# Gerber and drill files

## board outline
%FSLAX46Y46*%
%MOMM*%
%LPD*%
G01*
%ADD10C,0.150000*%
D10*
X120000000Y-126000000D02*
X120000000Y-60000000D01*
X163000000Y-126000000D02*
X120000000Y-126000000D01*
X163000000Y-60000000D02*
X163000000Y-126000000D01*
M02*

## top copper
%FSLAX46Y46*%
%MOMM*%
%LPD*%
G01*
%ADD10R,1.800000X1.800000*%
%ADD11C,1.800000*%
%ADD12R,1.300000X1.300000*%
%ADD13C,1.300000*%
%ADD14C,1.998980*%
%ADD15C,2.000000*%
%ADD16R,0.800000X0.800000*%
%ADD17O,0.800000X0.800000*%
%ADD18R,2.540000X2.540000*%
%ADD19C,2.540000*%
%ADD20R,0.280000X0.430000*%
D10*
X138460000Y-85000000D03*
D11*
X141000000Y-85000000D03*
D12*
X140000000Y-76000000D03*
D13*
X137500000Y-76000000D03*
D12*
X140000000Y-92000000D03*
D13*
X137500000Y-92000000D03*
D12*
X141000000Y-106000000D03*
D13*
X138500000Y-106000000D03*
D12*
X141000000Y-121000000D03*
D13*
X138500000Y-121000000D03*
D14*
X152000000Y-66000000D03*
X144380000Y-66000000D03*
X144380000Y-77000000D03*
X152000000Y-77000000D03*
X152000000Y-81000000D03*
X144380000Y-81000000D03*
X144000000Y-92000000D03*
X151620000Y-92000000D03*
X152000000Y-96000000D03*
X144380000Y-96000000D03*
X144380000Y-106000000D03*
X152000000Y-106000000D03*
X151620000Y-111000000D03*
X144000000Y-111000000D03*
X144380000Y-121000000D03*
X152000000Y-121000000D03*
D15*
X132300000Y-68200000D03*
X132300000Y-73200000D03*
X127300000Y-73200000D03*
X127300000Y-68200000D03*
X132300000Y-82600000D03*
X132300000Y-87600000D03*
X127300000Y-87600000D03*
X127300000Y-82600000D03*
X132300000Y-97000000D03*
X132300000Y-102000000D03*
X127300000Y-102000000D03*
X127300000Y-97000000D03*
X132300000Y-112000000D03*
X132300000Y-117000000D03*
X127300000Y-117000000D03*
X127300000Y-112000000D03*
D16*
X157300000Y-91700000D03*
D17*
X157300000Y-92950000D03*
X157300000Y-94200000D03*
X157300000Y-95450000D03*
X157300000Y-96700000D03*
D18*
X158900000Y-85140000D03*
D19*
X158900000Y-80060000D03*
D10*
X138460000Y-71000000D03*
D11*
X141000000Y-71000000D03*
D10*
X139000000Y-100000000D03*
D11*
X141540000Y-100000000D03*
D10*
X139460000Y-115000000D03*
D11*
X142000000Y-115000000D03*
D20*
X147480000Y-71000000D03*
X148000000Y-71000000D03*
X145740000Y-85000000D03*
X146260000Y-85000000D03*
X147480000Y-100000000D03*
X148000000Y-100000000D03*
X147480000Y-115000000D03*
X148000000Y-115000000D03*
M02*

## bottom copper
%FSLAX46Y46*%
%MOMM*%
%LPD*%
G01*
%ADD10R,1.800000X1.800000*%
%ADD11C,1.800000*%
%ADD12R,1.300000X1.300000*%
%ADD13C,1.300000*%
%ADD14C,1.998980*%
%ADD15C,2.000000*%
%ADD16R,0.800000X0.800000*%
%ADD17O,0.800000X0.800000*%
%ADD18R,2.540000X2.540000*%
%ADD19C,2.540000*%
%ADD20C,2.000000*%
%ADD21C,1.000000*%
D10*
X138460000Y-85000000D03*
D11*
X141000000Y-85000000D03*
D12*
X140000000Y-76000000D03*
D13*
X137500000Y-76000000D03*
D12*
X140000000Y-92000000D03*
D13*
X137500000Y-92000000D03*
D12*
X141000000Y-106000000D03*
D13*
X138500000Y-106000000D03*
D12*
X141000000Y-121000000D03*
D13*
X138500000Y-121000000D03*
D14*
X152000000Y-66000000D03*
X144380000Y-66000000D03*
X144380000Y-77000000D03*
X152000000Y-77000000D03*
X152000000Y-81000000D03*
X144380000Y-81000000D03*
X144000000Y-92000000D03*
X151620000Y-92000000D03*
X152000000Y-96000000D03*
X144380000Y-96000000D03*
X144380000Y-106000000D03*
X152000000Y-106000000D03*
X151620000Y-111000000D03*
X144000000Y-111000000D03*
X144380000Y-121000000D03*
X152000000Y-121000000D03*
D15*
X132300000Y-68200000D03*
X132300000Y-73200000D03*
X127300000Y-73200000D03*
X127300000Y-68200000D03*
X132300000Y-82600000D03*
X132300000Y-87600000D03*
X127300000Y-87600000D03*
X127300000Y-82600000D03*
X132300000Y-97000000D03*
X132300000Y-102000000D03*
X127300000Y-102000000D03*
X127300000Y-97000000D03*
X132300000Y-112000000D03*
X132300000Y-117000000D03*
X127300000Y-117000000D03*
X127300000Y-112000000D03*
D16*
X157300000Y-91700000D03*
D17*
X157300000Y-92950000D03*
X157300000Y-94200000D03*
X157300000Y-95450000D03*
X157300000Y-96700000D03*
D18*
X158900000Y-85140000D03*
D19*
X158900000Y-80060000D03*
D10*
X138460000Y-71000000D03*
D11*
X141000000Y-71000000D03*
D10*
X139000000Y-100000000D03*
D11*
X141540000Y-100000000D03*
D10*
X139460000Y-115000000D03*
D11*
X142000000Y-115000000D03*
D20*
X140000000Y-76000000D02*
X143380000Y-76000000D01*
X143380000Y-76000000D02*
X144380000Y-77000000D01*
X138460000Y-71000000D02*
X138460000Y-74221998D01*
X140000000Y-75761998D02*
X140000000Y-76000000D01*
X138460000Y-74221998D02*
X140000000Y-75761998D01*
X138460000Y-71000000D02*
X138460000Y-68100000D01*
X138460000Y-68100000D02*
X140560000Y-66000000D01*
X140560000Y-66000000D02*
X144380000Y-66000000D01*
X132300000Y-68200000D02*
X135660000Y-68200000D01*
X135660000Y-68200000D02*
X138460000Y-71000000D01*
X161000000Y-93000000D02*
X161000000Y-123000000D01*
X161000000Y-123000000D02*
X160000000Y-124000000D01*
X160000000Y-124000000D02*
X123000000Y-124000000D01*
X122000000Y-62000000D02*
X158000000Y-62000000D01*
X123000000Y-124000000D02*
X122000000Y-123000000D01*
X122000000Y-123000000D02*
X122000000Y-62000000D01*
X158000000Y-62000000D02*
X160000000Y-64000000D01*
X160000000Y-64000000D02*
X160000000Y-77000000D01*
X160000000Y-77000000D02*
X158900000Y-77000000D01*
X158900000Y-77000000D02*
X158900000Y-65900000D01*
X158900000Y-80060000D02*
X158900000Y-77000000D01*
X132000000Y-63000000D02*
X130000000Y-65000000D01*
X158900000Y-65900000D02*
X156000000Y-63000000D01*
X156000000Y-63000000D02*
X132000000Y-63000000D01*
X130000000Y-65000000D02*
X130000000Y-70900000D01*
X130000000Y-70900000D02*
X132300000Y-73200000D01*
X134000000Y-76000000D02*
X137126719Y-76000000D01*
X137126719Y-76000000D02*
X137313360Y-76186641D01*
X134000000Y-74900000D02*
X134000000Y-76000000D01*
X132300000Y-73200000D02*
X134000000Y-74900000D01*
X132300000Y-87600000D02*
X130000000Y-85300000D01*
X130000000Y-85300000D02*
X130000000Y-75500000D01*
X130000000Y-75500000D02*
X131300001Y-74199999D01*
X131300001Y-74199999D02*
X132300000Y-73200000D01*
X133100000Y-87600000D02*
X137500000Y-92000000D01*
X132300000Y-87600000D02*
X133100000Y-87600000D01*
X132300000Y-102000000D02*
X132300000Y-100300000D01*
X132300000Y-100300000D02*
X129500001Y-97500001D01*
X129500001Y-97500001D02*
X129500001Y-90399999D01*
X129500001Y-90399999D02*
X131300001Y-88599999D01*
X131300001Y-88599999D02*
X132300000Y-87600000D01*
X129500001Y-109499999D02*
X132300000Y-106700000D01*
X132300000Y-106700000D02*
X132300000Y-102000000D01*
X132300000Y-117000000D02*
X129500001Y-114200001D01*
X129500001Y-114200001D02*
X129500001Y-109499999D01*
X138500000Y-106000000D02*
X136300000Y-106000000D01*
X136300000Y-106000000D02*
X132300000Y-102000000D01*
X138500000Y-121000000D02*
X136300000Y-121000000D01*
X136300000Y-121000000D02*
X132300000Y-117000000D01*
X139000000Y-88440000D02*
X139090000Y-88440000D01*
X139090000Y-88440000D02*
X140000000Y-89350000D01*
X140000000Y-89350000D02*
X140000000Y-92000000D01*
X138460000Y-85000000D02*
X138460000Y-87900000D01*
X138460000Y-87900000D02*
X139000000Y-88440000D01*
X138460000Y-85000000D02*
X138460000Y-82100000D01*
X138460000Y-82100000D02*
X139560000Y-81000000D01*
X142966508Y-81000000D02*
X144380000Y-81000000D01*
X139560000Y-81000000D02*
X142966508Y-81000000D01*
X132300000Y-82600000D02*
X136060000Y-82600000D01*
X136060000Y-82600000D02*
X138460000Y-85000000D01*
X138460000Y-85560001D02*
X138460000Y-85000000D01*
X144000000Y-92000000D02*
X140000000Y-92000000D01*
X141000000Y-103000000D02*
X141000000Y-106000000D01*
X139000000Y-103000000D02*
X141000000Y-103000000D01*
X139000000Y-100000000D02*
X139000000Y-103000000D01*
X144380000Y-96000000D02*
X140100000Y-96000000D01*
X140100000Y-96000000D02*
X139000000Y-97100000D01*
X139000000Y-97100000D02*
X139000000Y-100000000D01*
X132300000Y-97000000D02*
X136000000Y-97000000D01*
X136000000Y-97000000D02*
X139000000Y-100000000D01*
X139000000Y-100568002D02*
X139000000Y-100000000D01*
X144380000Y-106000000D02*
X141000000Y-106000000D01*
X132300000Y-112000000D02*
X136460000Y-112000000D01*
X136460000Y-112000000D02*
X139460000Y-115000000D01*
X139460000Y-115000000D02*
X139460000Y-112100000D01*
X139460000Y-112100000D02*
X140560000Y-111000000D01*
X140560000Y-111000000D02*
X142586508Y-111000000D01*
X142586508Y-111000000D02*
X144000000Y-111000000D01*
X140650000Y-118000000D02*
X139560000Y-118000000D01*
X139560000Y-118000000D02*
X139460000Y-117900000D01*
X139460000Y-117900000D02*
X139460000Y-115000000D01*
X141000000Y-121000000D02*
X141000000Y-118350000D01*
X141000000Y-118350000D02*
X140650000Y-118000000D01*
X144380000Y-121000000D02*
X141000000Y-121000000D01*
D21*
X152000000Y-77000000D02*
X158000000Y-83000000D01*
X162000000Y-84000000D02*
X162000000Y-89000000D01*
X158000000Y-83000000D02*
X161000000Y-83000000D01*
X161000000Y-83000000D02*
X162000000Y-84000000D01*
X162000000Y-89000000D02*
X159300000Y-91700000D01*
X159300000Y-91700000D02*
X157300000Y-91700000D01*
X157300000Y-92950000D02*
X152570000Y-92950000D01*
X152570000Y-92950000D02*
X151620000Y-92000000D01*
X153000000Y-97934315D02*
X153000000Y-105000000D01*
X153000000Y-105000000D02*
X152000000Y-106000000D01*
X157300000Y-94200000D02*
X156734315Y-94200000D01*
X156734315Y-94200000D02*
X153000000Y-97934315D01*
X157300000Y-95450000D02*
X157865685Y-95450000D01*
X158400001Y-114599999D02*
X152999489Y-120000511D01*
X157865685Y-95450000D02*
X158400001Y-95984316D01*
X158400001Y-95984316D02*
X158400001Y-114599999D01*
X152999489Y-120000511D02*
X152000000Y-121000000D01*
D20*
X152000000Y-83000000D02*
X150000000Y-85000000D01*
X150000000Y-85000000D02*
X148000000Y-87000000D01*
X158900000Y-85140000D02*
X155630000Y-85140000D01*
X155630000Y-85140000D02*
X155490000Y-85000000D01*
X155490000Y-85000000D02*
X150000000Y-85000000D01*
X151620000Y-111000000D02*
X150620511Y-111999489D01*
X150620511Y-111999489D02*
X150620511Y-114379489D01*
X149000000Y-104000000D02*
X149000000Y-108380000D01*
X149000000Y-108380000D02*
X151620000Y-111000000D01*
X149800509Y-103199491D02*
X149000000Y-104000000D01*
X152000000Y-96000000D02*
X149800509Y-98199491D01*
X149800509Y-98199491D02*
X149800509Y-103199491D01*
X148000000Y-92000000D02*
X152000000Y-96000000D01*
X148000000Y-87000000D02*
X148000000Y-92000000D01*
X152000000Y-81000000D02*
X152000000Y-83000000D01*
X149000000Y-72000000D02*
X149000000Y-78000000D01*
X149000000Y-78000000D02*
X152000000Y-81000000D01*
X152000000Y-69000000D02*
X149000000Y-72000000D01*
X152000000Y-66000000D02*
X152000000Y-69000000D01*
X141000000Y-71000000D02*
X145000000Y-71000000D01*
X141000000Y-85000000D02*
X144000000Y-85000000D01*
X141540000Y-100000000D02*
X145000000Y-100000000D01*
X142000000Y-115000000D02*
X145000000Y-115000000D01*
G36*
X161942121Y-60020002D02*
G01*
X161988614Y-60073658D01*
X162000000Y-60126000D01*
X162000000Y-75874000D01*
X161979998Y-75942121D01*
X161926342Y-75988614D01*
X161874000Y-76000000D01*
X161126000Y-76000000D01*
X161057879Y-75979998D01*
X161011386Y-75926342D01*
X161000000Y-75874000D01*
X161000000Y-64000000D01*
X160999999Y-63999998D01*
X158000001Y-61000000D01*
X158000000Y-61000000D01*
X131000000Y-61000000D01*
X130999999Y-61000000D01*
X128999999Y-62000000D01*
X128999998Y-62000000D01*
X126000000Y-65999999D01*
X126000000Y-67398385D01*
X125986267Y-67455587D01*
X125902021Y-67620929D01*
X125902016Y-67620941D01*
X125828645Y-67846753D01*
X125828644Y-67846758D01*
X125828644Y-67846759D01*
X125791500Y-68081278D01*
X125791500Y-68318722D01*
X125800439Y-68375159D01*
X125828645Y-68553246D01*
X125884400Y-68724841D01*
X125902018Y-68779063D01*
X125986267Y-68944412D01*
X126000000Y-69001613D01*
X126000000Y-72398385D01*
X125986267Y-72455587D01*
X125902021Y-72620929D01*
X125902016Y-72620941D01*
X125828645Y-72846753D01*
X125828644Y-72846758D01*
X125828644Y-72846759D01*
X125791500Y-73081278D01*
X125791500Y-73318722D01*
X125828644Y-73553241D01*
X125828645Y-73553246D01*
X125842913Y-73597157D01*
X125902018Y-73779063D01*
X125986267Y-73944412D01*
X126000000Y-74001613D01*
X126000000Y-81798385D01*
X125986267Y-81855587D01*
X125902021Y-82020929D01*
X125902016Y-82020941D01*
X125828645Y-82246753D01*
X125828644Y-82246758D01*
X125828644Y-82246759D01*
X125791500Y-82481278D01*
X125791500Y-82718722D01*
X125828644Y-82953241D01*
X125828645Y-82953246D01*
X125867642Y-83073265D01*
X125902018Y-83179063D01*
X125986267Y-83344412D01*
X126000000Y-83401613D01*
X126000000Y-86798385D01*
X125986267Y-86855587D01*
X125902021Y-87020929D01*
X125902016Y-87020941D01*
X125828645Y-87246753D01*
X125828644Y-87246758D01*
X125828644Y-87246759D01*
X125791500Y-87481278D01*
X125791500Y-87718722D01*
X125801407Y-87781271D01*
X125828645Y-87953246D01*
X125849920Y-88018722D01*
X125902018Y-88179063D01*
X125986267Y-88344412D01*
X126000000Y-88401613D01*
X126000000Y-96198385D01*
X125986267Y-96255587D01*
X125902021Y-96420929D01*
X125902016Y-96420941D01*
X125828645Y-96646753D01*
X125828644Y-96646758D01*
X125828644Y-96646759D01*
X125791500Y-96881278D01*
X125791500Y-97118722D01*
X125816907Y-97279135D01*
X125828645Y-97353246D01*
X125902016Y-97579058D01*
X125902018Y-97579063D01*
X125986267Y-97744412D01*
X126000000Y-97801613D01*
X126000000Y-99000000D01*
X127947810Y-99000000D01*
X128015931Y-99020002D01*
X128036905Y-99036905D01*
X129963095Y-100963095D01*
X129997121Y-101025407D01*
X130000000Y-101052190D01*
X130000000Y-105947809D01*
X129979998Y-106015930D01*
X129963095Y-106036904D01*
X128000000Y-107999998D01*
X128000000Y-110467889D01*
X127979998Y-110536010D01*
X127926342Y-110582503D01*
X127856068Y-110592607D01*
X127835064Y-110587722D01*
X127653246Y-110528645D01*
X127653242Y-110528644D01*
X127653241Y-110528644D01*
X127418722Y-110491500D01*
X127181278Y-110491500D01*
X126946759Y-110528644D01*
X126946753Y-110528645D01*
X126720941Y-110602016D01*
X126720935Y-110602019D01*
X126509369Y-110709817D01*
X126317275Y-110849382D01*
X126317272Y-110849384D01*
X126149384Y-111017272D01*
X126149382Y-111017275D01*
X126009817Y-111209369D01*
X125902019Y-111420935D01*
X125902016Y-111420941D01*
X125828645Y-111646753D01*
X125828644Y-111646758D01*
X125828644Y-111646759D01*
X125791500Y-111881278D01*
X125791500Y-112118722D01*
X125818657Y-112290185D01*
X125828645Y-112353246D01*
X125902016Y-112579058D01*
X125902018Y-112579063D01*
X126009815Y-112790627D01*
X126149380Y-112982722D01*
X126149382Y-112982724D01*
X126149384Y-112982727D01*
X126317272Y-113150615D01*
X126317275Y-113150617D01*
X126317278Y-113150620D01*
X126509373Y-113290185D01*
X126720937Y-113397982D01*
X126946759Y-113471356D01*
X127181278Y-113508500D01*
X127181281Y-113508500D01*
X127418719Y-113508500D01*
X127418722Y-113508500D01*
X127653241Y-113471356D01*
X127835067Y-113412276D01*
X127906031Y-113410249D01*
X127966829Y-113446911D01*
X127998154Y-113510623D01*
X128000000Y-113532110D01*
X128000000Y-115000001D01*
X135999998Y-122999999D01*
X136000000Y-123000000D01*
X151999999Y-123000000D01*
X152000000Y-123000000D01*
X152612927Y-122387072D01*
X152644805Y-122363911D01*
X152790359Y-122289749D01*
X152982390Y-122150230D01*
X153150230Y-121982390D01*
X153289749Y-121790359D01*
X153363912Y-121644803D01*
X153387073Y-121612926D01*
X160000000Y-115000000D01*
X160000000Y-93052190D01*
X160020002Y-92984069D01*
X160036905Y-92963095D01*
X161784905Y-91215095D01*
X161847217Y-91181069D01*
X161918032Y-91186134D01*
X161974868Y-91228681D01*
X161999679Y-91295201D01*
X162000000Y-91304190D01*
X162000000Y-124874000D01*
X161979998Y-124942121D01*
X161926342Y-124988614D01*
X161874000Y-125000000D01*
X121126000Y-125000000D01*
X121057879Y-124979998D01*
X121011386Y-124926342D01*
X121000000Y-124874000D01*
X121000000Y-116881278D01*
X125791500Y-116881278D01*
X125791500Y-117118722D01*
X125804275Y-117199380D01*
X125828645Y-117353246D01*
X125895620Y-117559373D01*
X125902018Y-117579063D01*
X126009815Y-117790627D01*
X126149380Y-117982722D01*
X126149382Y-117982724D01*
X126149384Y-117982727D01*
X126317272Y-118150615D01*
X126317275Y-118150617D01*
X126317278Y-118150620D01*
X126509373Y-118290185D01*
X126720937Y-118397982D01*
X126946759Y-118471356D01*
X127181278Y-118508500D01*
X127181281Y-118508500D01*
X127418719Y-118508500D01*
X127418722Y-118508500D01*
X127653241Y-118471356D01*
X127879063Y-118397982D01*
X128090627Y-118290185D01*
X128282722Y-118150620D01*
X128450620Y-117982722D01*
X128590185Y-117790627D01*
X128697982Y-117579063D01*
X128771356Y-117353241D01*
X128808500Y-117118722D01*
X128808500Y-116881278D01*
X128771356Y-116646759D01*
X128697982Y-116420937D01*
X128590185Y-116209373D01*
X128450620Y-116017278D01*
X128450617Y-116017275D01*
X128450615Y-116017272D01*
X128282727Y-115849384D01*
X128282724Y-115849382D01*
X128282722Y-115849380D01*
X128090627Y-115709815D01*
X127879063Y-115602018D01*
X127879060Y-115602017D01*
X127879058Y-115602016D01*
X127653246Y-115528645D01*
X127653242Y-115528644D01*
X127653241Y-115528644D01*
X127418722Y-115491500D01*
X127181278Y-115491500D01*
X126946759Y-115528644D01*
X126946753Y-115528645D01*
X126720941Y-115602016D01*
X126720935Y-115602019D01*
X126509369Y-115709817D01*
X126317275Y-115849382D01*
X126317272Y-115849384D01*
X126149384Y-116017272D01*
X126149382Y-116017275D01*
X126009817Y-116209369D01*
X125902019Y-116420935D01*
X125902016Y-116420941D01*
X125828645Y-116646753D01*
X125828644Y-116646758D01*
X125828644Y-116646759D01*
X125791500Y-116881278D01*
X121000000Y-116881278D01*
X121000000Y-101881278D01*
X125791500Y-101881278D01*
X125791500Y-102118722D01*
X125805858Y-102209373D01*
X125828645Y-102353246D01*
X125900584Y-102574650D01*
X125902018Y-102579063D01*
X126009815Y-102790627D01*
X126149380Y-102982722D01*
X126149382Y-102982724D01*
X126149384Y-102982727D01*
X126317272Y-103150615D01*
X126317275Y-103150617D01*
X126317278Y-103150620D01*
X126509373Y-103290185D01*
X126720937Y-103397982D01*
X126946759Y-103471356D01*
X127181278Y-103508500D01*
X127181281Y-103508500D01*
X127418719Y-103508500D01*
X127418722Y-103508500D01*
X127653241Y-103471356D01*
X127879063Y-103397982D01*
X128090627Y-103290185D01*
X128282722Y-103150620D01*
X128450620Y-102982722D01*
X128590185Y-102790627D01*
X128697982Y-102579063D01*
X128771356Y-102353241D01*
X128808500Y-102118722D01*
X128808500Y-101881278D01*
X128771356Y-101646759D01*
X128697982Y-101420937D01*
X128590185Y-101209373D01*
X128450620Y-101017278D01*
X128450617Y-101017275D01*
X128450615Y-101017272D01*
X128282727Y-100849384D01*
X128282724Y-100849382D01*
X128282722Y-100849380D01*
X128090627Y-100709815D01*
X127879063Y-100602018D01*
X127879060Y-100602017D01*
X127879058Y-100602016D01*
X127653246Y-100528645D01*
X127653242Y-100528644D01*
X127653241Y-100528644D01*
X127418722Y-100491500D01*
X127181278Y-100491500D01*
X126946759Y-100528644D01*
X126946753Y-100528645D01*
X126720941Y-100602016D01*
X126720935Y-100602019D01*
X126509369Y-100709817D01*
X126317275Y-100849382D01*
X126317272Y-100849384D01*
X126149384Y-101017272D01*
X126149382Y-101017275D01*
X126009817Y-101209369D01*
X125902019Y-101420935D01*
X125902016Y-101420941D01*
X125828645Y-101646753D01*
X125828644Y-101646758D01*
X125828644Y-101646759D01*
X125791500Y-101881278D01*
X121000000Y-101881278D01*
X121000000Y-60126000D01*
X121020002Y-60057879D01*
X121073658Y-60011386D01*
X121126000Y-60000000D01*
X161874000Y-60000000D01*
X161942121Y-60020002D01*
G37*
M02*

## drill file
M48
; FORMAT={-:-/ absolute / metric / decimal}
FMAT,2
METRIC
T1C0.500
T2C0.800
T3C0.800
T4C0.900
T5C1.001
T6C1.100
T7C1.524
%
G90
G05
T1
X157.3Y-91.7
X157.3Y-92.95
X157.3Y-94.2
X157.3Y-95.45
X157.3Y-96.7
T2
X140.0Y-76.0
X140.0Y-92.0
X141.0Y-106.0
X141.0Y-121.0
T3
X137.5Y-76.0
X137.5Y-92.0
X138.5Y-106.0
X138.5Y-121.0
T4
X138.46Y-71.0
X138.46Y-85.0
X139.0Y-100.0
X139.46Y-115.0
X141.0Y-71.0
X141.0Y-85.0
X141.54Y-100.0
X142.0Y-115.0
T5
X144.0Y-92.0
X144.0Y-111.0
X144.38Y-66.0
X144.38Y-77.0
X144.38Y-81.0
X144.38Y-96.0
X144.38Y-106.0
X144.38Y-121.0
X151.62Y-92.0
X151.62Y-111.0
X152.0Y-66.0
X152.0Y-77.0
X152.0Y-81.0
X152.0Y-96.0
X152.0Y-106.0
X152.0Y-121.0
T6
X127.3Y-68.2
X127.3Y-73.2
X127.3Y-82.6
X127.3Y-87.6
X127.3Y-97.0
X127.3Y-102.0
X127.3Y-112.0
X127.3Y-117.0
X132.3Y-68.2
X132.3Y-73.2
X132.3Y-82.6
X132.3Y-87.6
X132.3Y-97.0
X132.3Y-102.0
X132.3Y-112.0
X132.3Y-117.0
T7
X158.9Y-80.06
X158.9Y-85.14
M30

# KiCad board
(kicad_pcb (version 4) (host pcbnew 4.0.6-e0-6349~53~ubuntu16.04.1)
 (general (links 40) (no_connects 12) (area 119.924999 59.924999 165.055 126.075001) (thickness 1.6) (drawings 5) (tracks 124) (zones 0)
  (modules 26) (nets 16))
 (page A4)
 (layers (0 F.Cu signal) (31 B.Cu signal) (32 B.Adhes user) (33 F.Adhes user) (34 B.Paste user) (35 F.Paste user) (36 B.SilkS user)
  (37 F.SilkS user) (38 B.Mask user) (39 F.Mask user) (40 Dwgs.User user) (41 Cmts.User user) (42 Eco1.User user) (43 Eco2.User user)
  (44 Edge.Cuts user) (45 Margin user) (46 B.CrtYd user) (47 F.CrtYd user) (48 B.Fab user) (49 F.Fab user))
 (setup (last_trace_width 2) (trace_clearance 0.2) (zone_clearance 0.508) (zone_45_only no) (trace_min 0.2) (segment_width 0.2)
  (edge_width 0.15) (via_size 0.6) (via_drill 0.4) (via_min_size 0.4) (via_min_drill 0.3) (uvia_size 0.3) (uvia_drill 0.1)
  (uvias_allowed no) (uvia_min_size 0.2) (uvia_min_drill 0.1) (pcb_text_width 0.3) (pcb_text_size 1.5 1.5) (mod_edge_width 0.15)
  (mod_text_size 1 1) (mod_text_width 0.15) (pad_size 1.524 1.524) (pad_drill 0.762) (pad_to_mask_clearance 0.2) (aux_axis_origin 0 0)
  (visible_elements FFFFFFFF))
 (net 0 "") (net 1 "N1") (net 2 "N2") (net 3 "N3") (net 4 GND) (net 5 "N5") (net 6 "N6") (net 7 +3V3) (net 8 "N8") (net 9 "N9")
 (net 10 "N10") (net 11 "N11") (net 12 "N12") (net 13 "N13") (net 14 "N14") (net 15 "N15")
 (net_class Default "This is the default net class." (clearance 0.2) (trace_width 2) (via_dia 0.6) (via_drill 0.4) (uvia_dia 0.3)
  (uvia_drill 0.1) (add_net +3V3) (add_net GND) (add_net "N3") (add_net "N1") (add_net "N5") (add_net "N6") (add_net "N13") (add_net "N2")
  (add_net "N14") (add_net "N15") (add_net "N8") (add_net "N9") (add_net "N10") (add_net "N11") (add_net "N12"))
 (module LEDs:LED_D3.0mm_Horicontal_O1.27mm (layer F.Cu) (at 138.46 85)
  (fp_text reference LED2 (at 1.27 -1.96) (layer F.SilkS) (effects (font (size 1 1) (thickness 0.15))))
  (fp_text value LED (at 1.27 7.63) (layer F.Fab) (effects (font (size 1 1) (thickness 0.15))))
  (pad 1 thru_hole rect (at 0 0) (size 1.8 1.8) (drill 0.9) (layers *.Cu *.Mask) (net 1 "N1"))
  (pad 2 thru_hole circle (at 2.54 0) (size 1.8 1.8) (drill 0.9) (layers *.Cu *.Mask) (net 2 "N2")))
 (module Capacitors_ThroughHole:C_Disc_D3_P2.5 (layer F.Cu) (at 140 76 180)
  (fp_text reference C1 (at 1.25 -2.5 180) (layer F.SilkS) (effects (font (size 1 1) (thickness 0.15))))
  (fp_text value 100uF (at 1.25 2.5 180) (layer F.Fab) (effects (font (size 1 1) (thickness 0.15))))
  (pad 1 thru_hole rect (at 0 0 180) (size 1.3 1.3) (drill 0.8) (layers *.Cu *.Mask F.SilkS) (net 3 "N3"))
  (pad 2 thru_hole circle (at 2.5 0 180) (size 1.3 1.3) (drill 0.8001) (layers *.Cu *.Mask F.SilkS) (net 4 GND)))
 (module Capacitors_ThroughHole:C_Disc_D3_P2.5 (layer F.Cu) (at 140 92 180)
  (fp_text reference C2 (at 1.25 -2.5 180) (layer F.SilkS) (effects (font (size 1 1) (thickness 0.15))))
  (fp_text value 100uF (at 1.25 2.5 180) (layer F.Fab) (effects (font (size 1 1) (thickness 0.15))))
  (pad 1 thru_hole rect (at 0 0 180) (size 1.3 1.3) (drill 0.8) (layers *.Cu *.Mask F.SilkS) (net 1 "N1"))
  (pad 2 thru_hole circle (at 2.5 0 180) (size 1.3 1.3) (drill 0.8001) (layers *.Cu *.Mask F.SilkS) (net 4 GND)))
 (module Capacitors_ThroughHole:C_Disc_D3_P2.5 (layer F.Cu) (at 141 106 180)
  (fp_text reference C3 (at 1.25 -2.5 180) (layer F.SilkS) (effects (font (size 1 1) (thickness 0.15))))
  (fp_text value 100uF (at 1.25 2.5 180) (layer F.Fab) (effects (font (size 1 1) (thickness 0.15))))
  (pad 1 thru_hole rect (at 0 0 180) (size 1.3 1.3) (drill 0.8) (layers *.Cu *.Mask F.SilkS) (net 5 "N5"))
  (pad 2 thru_hole circle (at 2.5 0 180) (size 1.3 1.3) (drill 0.8001) (layers *.Cu *.Mask F.SilkS) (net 4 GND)))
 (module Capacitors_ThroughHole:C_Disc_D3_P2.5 (layer F.Cu) (at 141 121 180)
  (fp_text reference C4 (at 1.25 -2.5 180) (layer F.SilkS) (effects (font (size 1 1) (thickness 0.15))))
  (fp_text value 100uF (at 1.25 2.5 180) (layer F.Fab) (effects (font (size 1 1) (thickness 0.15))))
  (pad 1 thru_hole rect (at 0 0 180) (size 1.3 1.3) (drill 0.8) (layers *.Cu *.Mask F.SilkS) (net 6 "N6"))
  (pad 2 thru_hole circle (at 2.5 0 180) (size 1.3 1.3) (drill 0.8001) (layers *.Cu *.Mask F.SilkS) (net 4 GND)))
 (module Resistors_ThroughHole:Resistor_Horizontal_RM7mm (layer F.Cu) (at 152 66 180)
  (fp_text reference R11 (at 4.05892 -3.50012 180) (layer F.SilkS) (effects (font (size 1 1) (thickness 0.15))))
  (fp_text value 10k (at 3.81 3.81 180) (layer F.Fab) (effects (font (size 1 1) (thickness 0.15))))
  (pad 1 thru_hole circle (at 0 0 180) (size 1.99898 1.99898) (drill 1.00076) (layers *.Cu *.SilkS *.Mask) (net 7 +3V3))
  (pad 2 thru_hole circle (at 7.62 0 180) (size 1.99898 1.99898) (drill 1.00076) (layers *.Cu *.SilkS *.Mask) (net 3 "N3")))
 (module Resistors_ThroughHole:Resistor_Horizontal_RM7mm (layer F.Cu) (at 144.38 77)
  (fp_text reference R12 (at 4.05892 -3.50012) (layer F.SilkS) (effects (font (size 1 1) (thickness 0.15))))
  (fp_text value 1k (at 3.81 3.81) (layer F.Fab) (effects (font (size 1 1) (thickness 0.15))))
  (pad 1 thru_hole circle (at 0 0) (size 1.99898 1.99898) (drill 1.00076) (layers *.Cu *.SilkS *.Mask) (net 3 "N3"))
  (pad 2 thru_hole circle (at 7.62 0) (size 1.99898 1.99898) (drill 1.00076) (layers *.Cu *.SilkS *.Mask) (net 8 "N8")))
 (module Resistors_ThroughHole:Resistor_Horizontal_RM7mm (layer F.Cu) (at 152 81 180)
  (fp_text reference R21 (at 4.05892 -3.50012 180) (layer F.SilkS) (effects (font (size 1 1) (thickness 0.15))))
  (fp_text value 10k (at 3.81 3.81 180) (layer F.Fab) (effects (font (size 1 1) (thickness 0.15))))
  (pad 1 thru_hole circle (at 0 0 180) (size 1.99898 1.99898) (drill 1.00076) (layers *.Cu *.SilkS *.Mask) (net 7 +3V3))
  (pad 2 thru_hole circle (at 7.62 0 180) (size 1.99898 1.99898) (drill 1.00076) (layers *.Cu *.SilkS *.Mask) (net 1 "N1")))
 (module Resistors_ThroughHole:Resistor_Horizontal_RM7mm (layer F.Cu) (at 144 92)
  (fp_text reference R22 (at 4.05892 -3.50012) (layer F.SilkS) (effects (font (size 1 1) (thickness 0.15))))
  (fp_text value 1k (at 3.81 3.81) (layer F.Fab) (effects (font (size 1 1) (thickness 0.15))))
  (pad 1 thru_hole circle (at 0 0) (size 1.99898 1.99898) (drill 1.00076) (layers *.Cu *.SilkS *.Mask) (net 1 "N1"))
  (pad 2 thru_hole circle (at 7.62 0) (size 1.99898 1.99898) (drill 1.00076) (layers *.Cu *.SilkS *.Mask) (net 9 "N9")))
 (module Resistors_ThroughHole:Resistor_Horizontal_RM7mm (layer F.Cu) (at 152 96 180)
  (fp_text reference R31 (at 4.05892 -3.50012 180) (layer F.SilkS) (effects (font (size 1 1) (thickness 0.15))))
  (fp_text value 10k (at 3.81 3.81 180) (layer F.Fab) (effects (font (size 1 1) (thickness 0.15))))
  (pad 1 thru_hole circle (at 0 0 180) (size 1.99898 1.99898) (drill 1.00076) (layers *.Cu *.SilkS *.Mask) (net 7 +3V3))
  (pad 2 thru_hole circle (at 7.62 0 180) (size 1.99898 1.99898) (drill 1.00076) (layers *.Cu *.SilkS *.Mask) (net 5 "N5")))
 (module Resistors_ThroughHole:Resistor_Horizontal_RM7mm (layer F.Cu) (at 144.38 106)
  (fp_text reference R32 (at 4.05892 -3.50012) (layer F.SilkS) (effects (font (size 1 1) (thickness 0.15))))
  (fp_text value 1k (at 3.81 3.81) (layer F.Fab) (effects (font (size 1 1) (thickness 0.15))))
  (pad 1 thru_hole circle (at 0 0) (size 1.99898 1.99898) (drill 1.00076) (layers *.Cu *.SilkS *.Mask) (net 5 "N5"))
  (pad 2 thru_hole circle (at 7.62 0) (size 1.99898 1.99898) (drill 1.00076) (layers *.Cu *.SilkS *.Mask) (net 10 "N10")))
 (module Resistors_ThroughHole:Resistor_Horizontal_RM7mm (layer F.Cu) (at 151.62 111 180)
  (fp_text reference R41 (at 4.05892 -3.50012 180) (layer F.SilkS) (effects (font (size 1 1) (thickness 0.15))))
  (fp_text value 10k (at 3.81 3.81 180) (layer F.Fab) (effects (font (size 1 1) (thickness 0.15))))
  (pad 1 thru_hole circle (at 0 0 180) (size 1.99898 1.99898) (drill 1.00076) (layers *.Cu *.SilkS *.Mask) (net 7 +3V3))
  (pad 2 thru_hole circle (at 7.62 0 180) (size 1.99898 1.99898) (drill 1.00076) (layers *.Cu *.SilkS *.Mask) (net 6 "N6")))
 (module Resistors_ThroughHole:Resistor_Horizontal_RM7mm (layer F.Cu) (at 144.38 121)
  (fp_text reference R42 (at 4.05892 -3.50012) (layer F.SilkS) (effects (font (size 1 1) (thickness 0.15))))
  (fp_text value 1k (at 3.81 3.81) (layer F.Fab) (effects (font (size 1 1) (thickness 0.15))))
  (pad 1 thru_hole circle (at 0 0) (size 1.99898 1.99898) (drill 1.00076) (layers *.Cu *.SilkS *.Mask) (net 6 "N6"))
  (pad 2 thru_hole circle (at 7.62 0) (size 1.99898 1.99898) (drill 1.00076) (layers *.Cu *.SilkS *.Mask) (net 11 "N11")))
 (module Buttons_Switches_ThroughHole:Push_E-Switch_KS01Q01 (layer F.Cu) (at 132.3 68.2 270)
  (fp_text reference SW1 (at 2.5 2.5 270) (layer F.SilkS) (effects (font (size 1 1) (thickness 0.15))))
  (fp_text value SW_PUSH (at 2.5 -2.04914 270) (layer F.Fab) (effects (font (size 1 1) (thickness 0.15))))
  (pad 1 thru_hole circle (at 0 0 270) (size 2 2) (drill 1.1) (layers *.Cu *.Mask F.SilkS) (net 3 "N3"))
  (pad 2 thru_hole circle (at 5 0 270) (size 2 2) (drill 1.1) (layers *.Cu *.Mask F.SilkS) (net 4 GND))
  (pad 4 thru_hole circle (at 5 5 270) (size 2 2) (drill 1.1) (layers *.Cu *.Mask F.SilkS))
  (pad 3 thru_hole circle (at 0 5 270) (size 2 2) (drill 1.1) (layers *.Cu *.Mask F.SilkS)))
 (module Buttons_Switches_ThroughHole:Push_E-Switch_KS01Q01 (layer F.Cu) (at 132.3 82.6 270)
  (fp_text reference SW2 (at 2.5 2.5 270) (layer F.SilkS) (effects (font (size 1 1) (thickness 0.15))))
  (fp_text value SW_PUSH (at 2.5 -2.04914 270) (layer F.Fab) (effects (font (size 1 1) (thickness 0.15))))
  (pad 1 thru_hole circle (at 0 0 270) (size 2 2) (drill 1.1) (layers *.Cu *.Mask F.SilkS) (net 1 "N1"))
  (pad 2 thru_hole circle (at 5 0 270) (size 2 2) (drill 1.1) (layers *.Cu *.Mask F.SilkS) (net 4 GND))
  (pad 4 thru_hole circle (at 5 5 270) (size 2 2) (drill 1.1) (layers *.Cu *.Mask F.SilkS))
  (pad 3 thru_hole circle (at 0 5 270) (size 2 2) (drill 1.1) (layers *.Cu *.Mask F.SilkS)))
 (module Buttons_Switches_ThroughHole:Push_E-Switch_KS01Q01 (layer F.Cu) (at 132.3 97 270)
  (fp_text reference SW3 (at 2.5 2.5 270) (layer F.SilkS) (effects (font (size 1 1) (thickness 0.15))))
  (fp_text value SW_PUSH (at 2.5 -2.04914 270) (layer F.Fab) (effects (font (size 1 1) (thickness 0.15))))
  (pad 1 thru_hole circle (at 0 0 270) (size 2 2) (drill 1.1) (layers *.Cu *.Mask F.SilkS) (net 5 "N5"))
  (pad 2 thru_hole circle (at 5 0 270) (size 2 2) (drill 1.1) (layers *.Cu *.Mask F.SilkS) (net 4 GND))
  (pad 4 thru_hole circle (at 5 5 270) (size 2 2) (drill 1.1) (layers *.Cu *.Mask F.SilkS))
  (pad 3 thru_hole circle (at 0 5 270) (size 2 2) (drill 1.1) (layers *.Cu *.Mask F.SilkS)))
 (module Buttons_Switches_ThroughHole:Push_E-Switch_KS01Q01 (layer F.Cu) (at 132.3 112 270)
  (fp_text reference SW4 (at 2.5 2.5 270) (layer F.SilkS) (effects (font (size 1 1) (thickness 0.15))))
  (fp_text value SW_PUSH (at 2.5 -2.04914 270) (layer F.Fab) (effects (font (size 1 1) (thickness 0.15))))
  (pad 1 thru_hole circle (at 0 0 270) (size 2 2) (drill 1.1) (layers *.Cu *.Mask F.SilkS) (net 6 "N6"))
  (pad 2 thru_hole circle (at 5 0 270) (size 2 2) (drill 1.1) (layers *.Cu *.Mask F.SilkS) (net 4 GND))
  (pad 4 thru_hole circle (at 5 5 270) (size 2 2) (drill 1.1) (layers *.Cu *.Mask F.SilkS))
  (pad 3 thru_hole circle (at 0 5 270) (size 2 2) (drill 1.1) (layers *.Cu *.Mask F.SilkS)))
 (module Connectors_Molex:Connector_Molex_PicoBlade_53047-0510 (layer F.Cu) (at 157.3 91.7 270)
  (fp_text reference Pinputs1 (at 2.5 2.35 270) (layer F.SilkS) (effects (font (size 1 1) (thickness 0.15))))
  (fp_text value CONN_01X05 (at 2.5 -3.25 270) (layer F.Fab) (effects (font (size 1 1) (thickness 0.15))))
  (pad 1 thru_hole rect (at 0 0 270) (size 0.8 0.8) (drill 0.5) (layers *.Cu *.Mask F.SilkS) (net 8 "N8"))
  (pad 2 thru_hole oval (at 1.25 0 270) (size 0.8 0.8) (drill 0.5) (layers *.Cu *.Mask F.SilkS) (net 9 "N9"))
  (pad 3 thru_hole oval (at 2.5 0 270) (size 0.8 0.8) (drill 0.5) (layers *.Cu *.Mask F.SilkS) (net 10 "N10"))
  (pad 4 thru_hole oval (at 3.75 0 270) (size 0.8 0.8) (drill 0.5) (layers *.Cu *.Mask F.SilkS) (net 11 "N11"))
  (pad 5 thru_hole oval (at 5 0 270) (size 0.8 0.8) (drill 0.5) (layers *.Cu *.Mask F.SilkS) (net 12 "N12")))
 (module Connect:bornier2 (layer F.Cu) (at 158.9 82.6 90)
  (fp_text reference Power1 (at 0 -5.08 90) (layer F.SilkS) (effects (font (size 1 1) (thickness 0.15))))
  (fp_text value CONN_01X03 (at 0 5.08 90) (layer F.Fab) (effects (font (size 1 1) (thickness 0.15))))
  (pad 1 thru_hole rect (at -2.54 0 90) (size 2.54 2.54) (drill 1.524) (layers *.Cu *.Mask F.SilkS) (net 7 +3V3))
  (pad 2 thru_hole circle (at 2.54 0 90) (size 2.54 2.54) (drill 1.524) (layers *.Cu *.Mask F.SilkS) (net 4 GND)))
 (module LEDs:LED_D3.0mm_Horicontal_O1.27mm (layer F.Cu) (at 138.46 71)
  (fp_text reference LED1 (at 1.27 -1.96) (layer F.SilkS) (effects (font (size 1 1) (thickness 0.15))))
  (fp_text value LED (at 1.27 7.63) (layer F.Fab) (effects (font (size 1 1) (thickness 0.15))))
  (pad 1 thru_hole rect (at 0 0) (size 1.8 1.8) (drill 0.9) (layers *.Cu *.Mask) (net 3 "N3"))
  (pad 2 thru_hole circle (at 2.54 0) (size 1.8 1.8) (drill 0.9) (layers *.Cu *.Mask) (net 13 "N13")))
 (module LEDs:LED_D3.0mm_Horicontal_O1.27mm (layer F.Cu) (at 139 100)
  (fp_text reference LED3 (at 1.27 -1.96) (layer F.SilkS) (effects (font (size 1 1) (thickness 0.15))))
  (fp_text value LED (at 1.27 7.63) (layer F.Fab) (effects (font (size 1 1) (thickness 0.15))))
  (pad 1 thru_hole rect (at 0 0) (size 1.8 1.8) (drill 0.9) (layers *.Cu *.Mask) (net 5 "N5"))
  (pad 2 thru_hole circle (at 2.54 0) (size 1.8 1.8) (drill 0.9) (layers *.Cu *.Mask) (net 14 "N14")))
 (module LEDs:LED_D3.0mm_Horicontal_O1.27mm (layer F.Cu) (at 139.46 115)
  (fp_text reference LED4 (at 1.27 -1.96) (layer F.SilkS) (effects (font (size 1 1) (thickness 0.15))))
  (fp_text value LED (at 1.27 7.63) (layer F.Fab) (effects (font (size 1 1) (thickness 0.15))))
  (pad 1 thru_hole rect (at 0 0) (size 1.8 1.8) (drill 0.9) (layers *.Cu *.Mask) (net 6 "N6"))
  (pad 2 thru_hole circle (at 2.54 0) (size 1.8 1.8) (drill 0.9) (layers *.Cu *.Mask) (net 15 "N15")))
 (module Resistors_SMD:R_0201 (layer F.Cu) (at 147.74 71)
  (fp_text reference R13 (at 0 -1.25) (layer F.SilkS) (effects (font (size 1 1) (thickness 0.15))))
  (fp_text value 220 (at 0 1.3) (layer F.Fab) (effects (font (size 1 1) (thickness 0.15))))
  (pad 1 smd rect (at -0.26 0) (size 0.28 0.43) (layers F.Cu F.Paste F.Mask) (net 13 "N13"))
  (pad 2 smd rect (at 0.26 0) (size 0.28 0.43) (layers F.Cu F.Paste F.Mask) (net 7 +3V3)))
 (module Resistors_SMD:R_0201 (layer F.Cu) (at 146 85)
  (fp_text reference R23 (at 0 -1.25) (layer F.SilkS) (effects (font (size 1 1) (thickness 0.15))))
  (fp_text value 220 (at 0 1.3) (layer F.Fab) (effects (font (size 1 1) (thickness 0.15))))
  (pad 1 smd rect (at -0.26 0) (size 0.28 0.43) (layers F.Cu F.Paste F.Mask) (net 2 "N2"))
  (pad 2 smd rect (at 0.26 0) (size 0.28 0.43) (layers F.Cu F.Paste F.Mask) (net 7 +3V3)))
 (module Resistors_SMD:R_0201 (layer F.Cu) (at 147.74 100)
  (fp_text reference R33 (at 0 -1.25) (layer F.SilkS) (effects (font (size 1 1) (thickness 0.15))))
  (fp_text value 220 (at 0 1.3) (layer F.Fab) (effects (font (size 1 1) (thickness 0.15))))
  (pad 1 smd rect (at -0.26 0) (size 0.28 0.43) (layers F.Cu F.Paste F.Mask) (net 14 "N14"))
  (pad 2 smd rect (at 0.26 0) (size 0.28 0.43) (layers F.Cu F.Paste F.Mask) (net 7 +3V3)))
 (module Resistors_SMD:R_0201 (layer F.Cu) (at 147.74 115)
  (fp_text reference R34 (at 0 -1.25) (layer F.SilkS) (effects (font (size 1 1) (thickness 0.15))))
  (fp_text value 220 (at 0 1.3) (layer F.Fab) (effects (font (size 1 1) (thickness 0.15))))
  (pad 1 smd rect (at -0.26 0) (size 0.28 0.43) (layers F.Cu F.Paste F.Mask) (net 15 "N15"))
  (pad 2 smd rect (at 0.26 0) (size 0.28 0.43) (layers F.Cu F.Paste F.Mask) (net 7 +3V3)))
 (gr_line (start 120 126) (end 120 60) (layer Edge.Cuts) (width 0.15))
 (gr_line (start 163 126) (end 120 126) (layer Edge.Cuts) (width 0.15))
 (gr_line (start 163 60) (end 163 126) (layer Edge.Cuts) (width 0.15))
 (segment (start 140 76) (end 143.38 76) (width 2) (layer B.Cu) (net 3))
 (segment (start 143.38 76) (end 144.38 77) (width 2) (layer B.Cu) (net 3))
 (segment (start 138.46 71) (end 138.46 74.221998) (width 2) (layer B.Cu) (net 3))
 (segment (start 140 75.761998) (end 140 76) (width 2) (layer B.Cu) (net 3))
 (segment (start 138.46 74.221998) (end 140 75.761998) (width 2) (layer B.Cu) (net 3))
 (segment (start 138.46 71) (end 138.46 68.1) (width 2) (layer B.Cu) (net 3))
 (segment (start 138.46 68.1) (end 140.56 66) (width 2) (layer B.Cu) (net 3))
 (segment (start 140.56 66) (end 144.38 66) (width 2) (layer B.Cu) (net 3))
 (segment (start 132.3 68.2) (end 135.66 68.2) (width 2) (layer B.Cu) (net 3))
 (segment (start 135.66 68.2) (end 138.46 71) (width 2) (layer B.Cu) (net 3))
 (segment (start 161 93) (end 161 123) (width 2) (layer B.Cu) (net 4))
 (segment (start 161 123) (end 160 124) (width 2) (layer B.Cu) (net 4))
 (segment (start 160 124) (end 123 124) (width 2) (layer B.Cu) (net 4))
 (segment (start 122 62) (end 158 62) (width 2) (layer B.Cu) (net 4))
 (segment (start 123 124) (end 122 123) (width 2) (layer B.Cu) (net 4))
 (segment (start 122 123) (end 122 62) (width 2) (layer B.Cu) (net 4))
 (segment (start 158 62) (end 160 64) (width 2) (layer B.Cu) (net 4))
 (segment (start 160 64) (end 160 77) (width 2) (layer B.Cu) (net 4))
 (segment (start 160 77) (end 158.9 77) (width 2) (layer B.Cu) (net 4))
 (segment (start 158.9 77) (end 158.9 65.9) (width 2) (layer B.Cu) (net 4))
 (segment (start 158.9 80.06) (end 158.9 77) (width 2) (layer B.Cu) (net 4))
 (segment (start 132 63) (end 130 65) (width 2) (layer B.Cu) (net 4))
 (segment (start 158.9 65.9) (end 156 63) (width 2) (layer B.Cu) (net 4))
 (segment (start 156 63) (end 132 63) (width 2) (layer B.Cu) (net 4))
 (segment (start 130 65) (end 130 70.9) (width 2) (layer B.Cu) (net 4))
 (segment (start 130 70.9) (end 132.3 73.2) (width 2) (layer B.Cu) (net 4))
 (segment (start 134 76) (end 137.126719 76) (width 2) (layer B.Cu) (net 4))
 (segment (start 137.126719 76) (end 137.31336 76.186641) (width 2) (layer B.Cu) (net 4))
 (segment (start 134 74.9) (end 134 76) (width 2) (layer B.Cu) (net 4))
 (segment (start 132.3 73.2) (end 134 74.9) (width 2) (layer B.Cu) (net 4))
 (segment (start 132.3 87.6) (end 130 85.3) (width 2) (layer B.Cu) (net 4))
 (segment (start 130 85.3) (end 130 75.5) (width 2) (layer B.Cu) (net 4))
 (segment (start 130 75.5) (end 131.300001 74.199999) (width 2) (layer B.Cu) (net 4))
 (segment (start 131.300001 74.199999) (end 132.3 73.2) (width 2) (layer B.Cu) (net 4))
 (segment (start 133.1 87.6) (end 137.5 92) (width 2) (layer B.Cu) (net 4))
 (segment (start 132.3 87.6) (end 133.1 87.6) (width 2) (layer B.Cu) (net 4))
 (segment (start 132.3 102) (end 132.3 100.3) (width 2) (layer B.Cu) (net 4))
 (segment (start 132.3 100.3) (end 129.500001 97.500001) (width 2) (layer B.Cu) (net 4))
 (segment (start 129.500001 97.500001) (end 129.500001 90.399999) (width 2) (layer B.Cu) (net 4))
 (segment (start 129.500001 90.399999) (end 131.300001 88.599999) (width 2) (layer B.Cu) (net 4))
 (segment (start 131.300001 88.599999) (end 132.3 87.6) (width 2) (layer B.Cu) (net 4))
 (segment (start 129.500001 109.499999) (end 132.3 106.7) (width 2) (layer B.Cu) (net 4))
 (segment (start 132.3 106.7) (end 132.3 102) (width 2) (layer B.Cu) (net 4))
 (segment (start 132.3 117) (end 129.500001 114.200001) (width 2) (layer B.Cu) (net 4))
 (segment (start 129.500001 114.200001) (end 129.500001 109.499999) (width 2) (layer B.Cu) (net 4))
 (segment (start 138.5 106) (end 136.3 106) (width 2) (layer B.Cu) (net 4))
 (segment (start 136.3 106) (end 132.3 102) (width 2) (layer B.Cu) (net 4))
 (segment (start 138.5 121) (end 136.3 121) (width 2) (layer B.Cu) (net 4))
 (segment (start 136.3 121) (end 132.3 117) (width 2) (layer B.Cu) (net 4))
 (segment (start 139 88.44) (end 139.09 88.44) (width 2) (layer B.Cu) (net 1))
 (segment (start 139.09 88.44) (end 140 89.35) (width 2) (layer B.Cu) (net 1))
 (segment (start 140 89.35) (end 140 92) (width 2) (layer B.Cu) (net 1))
 (segment (start 138.46 85) (end 138.46 87.9) (width 2) (layer B.Cu) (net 1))
 (segment (start 138.46 87.9) (end 139 88.44) (width 2) (layer B.Cu) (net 1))
 (segment (start 138.46 85) (end 138.46 82.1) (width 2) (layer B.Cu) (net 1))
 (segment (start 138.46 82.1) (end 139.56 81) (width 2) (layer B.Cu) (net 1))
 (segment (start 142.966508 81) (end 144.38 81) (width 2) (layer B.Cu) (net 1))
 (segment (start 139.56 81) (end 142.966508 81) (width 2) (layer B.Cu) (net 1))
 (segment (start 132.3 82.6) (end 136.06 82.6) (width 2) (layer B.Cu) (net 1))
 (segment (start 136.06 82.6) (end 138.46 85) (width 2) (layer B.Cu) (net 1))
 (segment (start 138.46 85.560001) (end 138.46 85) (width 2) (layer B.Cu) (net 1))
 (segment (start 144 92) (end 140 92) (width 2) (layer B.Cu) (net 1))
 (segment (start 141 103) (end 141 106) (width 2) (layer B.Cu) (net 5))
 (segment (start 139 103) (end 141 103) (width 2) (layer B.Cu) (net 5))
 (segment (start 139 100) (end 139 103) (width 2) (layer B.Cu) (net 5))
 (segment (start 144.38 96) (end 140.1 96) (width 2) (layer B.Cu) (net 5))
 (segment (start 140.1 96) (end 139 97.1) (width 2) (layer B.Cu) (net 5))
 (segment (start 139 97.1) (end 139 100) (width 2) (layer B.Cu) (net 5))
 (segment (start 132.3 97) (end 136 97) (width 2) (layer B.Cu) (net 5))
 (segment (start 136 97) (end 139 100) (width 2) (layer B.Cu) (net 5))
 (segment (start 139 100.568002) (end 139 100) (width 2) (layer B.Cu) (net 5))
 (segment (start 144.38 106) (end 141 106) (width 2) (layer B.Cu) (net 5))
 (segment (start 132.3 112) (end 136.46 112) (width 2) (layer B.Cu) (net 6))
 (segment (start 136.46 112) (end 139.46 115) (width 2) (layer B.Cu) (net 6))
 (segment (start 139.46 115) (end 139.46 112.1) (width 2) (layer B.Cu) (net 6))
 (segment (start 139.46 112.1) (end 140.56 111) (width 2) (layer B.Cu) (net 6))
 (segment (start 140.56 111) (end 142.586508 111) (width 2) (layer B.Cu) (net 6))
 (segment (start 142.586508 111) (end 144 111) (width 2) (layer B.Cu) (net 6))
 (segment (start 140.65 118) (end 139.56 118) (width 2) (layer B.Cu) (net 6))
 (segment (start 139.56 118) (end 139.46 117.9) (width 2) (layer B.Cu) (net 6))
 (segment (start 139.46 117.9) (end 139.46 115) (width 2) (layer B.Cu) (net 6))
 (segment (start 141 121) (end 141 118.35) (width 2) (layer B.Cu) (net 6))
 (segment (start 141 118.35) (end 140.65 118) (width 2) (layer B.Cu) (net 6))
 (segment (start 144.38 121) (end 141 121) (width 2) (layer B.Cu) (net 6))
 (segment (start 152 77) (end 158 83) (width 1) (layer B.Cu) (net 8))
 (segment (start 162 84) (end 162 89) (width 1) (layer B.Cu) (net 8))
 (segment (start 158 83) (end 161 83) (width 1) (layer B.Cu) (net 8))
 (segment (start 161 83) (end 162 84) (width 1) (layer B.Cu) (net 8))
 (segment (start 162 89) (end 159.3 91.7) (width 1) (layer B.Cu) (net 8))
 (segment (start 159.3 91.7) (end 157.3 91.7) (width 1) (layer B.Cu) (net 8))
 (segment (start 157.3 92.95) (end 152.57 92.95) (width 1) (layer B.Cu) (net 9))
 (segment (start 152.57 92.95) (end 151.62 92) (width 1) (layer B.Cu) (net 9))
 (segment (start 153 97.934315) (end 153 105) (width 1) (layer B.Cu) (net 10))
 (segment (start 153 105) (end 152 106) (width 1) (layer B.Cu) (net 10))
 (segment (start 157.3 94.2) (end 156.734315 94.2) (width 1) (layer B.Cu) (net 10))
 (segment (start 156.734315 94.2) (end 153 97.934315) (width 1) (layer B.Cu) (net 10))
 (segment (start 157.3 95.45) (end 157.865685 95.45) (width 1) (layer B.Cu) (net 11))
 (segment (start 158.400001 114.599999) (end 152.999489 120.000511) (width 1) (layer B.Cu) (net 11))
 (segment (start 157.865685 95.45) (end 158.400001 95.984316) (width 1) (layer B.Cu) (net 11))
 (segment (start 158.400001 95.984316) (end 158.400001 114.599999) (width 1) (layer B.Cu) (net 11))
 (segment (start 152.999489 120.000511) (end 152 121) (width 1) (layer B.Cu) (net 11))
 (segment (start 152 83) (end 150 85) (width 2) (layer B.Cu) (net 7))
 (segment (start 150 85) (end 148 87) (width 2) (layer B.Cu) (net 7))
 (segment (start 158.9 85.14) (end 155.63 85.14) (width 2) (layer B.Cu) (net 7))
 (segment (start 155.63 85.14) (end 155.49 85) (width 2) (layer B.Cu) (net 7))
 (segment (start 155.49 85) (end 150 85) (width 2) (layer B.Cu) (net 7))
 (segment (start 151.62 111) (end 150.620511 111.999489) (width 2) (layer B.Cu) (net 7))
 (segment (start 150.620511 111.999489) (end 150.620511 114.379489) (width 2) (layer B.Cu) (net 7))
 (segment (start 149 104) (end 149 108.38) (width 2) (layer B.Cu) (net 7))
 (segment (start 149 108.38) (end 151.62 111) (width 2) (layer B.Cu) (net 7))
 (segment (start 149.800509 103.199491) (end 149 104) (width 2) (layer B.Cu) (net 7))
 (segment (start 152 96) (end 149.800509 98.199491) (width 2) (layer B.Cu) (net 7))
 (segment (start 149.800509 98.199491) (end 149.800509 103.199491) (width 2) (layer B.Cu) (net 7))
 (segment (start 148 92) (end 152 96) (width 2) (layer B.Cu) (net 7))
 (segment (start 148 87) (end 148 92) (width 2) (layer B.Cu) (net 7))
 (segment (start 152 81) (end 152 83) (width 2) (layer B.Cu) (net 7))
 (segment (start 149 72) (end 149 78) (width 2) (layer B.Cu) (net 7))
 (segment (start 149 78) (end 152 81) (width 2) (layer B.Cu) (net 7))
 (segment (start 152 69) (end 149 72) (width 2) (layer B.Cu) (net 7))
 (segment (start 152 66) (end 152 69) (width 2) (layer B.Cu) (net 7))
 (segment (start 141 71) (end 145 71) (width 2) (layer B.Cu) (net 13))
 (segment (start 141 85) (end 144 85) (width 2) (layer B.Cu) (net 2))
 (segment (start 141.54 100) (end 145 100) (width 2) (layer B.Cu) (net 14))
 (segment (start 142 115) (end 145 115) (width 2) (layer B.Cu) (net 15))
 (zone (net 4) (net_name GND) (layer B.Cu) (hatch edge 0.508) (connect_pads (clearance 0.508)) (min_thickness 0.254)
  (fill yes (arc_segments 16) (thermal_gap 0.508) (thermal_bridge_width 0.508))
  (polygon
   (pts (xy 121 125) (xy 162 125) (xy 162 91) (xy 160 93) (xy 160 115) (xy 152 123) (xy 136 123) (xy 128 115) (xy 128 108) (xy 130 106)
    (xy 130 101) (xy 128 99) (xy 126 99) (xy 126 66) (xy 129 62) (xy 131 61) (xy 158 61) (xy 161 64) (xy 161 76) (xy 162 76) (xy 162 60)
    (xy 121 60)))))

